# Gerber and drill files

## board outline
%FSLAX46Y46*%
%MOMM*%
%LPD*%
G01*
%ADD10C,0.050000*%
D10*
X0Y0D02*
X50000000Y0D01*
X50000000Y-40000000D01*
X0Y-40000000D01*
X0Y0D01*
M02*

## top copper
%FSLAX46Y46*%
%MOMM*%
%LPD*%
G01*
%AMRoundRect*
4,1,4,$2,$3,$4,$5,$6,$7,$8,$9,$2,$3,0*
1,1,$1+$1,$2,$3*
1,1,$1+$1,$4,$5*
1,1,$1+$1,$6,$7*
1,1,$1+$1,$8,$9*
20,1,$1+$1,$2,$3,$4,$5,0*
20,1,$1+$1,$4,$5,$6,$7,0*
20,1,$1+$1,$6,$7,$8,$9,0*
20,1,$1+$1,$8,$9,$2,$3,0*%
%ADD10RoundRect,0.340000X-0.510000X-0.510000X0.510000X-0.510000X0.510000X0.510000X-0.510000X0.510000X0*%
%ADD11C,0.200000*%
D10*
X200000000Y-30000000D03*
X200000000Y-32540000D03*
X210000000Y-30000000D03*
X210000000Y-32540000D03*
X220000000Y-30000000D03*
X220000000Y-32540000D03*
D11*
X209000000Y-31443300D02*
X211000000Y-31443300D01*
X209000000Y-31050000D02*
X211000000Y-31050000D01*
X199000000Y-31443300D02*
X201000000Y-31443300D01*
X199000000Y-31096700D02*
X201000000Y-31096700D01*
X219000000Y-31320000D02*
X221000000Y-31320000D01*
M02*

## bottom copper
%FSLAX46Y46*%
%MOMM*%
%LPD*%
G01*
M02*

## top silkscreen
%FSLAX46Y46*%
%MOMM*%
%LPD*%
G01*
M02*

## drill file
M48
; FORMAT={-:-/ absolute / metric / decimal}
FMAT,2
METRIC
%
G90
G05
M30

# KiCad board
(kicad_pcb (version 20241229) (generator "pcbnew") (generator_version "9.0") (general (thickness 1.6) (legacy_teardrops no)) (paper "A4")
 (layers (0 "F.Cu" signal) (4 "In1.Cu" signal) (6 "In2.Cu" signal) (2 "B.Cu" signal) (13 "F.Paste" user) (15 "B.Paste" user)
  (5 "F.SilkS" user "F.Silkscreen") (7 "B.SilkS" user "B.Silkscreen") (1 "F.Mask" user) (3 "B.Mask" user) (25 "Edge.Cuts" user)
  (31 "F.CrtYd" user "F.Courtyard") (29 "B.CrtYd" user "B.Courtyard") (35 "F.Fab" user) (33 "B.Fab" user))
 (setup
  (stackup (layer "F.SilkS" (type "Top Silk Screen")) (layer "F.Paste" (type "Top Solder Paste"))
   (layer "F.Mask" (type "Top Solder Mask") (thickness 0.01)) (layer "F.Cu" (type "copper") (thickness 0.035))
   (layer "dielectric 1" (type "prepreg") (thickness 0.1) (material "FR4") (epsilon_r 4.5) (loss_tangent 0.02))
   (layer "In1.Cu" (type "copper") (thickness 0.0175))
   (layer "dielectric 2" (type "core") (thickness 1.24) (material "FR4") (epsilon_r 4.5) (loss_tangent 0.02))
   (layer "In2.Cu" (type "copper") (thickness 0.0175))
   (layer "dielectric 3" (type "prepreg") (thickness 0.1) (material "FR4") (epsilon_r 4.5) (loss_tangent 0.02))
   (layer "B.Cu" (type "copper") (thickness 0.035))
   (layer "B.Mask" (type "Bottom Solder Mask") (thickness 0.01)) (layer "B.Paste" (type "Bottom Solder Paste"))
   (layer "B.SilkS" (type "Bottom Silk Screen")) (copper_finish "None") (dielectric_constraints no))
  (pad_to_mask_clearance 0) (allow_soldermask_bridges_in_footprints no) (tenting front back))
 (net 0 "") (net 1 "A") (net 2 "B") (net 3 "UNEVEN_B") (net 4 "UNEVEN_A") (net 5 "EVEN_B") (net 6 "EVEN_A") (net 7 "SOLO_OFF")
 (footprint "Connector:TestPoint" (layer "F.Cu") (at 200 30)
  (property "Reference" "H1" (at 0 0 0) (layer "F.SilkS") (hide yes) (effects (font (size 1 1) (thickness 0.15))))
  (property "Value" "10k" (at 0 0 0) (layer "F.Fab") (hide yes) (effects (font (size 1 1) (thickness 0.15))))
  (pad "1" smd roundrect (at 0 0) (size 1.7 1.7) (layers "F.Cu" "F.Paste" "F.Mask") (roundrect_rratio 0.2) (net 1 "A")))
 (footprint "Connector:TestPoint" (layer "F.Cu") (at 200 32.54)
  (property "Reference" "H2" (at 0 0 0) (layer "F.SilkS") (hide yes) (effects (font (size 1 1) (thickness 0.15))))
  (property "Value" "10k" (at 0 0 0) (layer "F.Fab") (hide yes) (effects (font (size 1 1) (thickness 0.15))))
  (pad "1" smd roundrect (at 0 0) (size 1.7 1.7) (layers "F.Cu" "F.Paste" "F.Mask") (roundrect_rratio 0.2) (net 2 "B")))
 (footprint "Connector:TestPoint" (layer "F.Cu") (at 210 30)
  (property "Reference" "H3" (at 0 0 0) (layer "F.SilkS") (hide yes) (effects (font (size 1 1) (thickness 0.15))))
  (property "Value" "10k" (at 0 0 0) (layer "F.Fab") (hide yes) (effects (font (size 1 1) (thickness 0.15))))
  (pad "1" smd roundrect (at 0 0) (size 1.7 1.7) (layers "F.Cu" "F.Paste" "F.Mask") (roundrect_rratio 0.2) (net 1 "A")))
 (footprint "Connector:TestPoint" (layer "F.Cu") (at 210 32.54)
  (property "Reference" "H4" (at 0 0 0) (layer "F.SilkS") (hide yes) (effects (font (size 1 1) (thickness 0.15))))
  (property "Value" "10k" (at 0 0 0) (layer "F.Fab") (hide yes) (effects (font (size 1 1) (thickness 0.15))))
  (pad "1" smd roundrect (at 0 0) (size 1.7 1.7) (layers "F.Cu" "F.Paste" "F.Mask") (roundrect_rratio 0.2) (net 2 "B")))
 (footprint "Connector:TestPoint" (layer "F.Cu") (at 220 30)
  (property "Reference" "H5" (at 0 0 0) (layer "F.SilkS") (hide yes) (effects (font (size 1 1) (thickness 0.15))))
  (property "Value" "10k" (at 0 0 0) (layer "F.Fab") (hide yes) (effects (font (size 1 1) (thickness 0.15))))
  (pad "1" smd roundrect (at 0 0) (size 1.7 1.7) (layers "F.Cu" "F.Paste" "F.Mask") (roundrect_rratio 0.2) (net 1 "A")))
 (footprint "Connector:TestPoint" (layer "F.Cu") (at 220 32.54)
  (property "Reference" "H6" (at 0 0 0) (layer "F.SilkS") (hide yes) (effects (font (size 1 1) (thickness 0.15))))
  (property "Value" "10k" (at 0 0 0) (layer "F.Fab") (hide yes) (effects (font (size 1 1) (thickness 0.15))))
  (pad "1" smd roundrect (at 0 0) (size 1.7 1.7) (layers "F.Cu" "F.Paste" "F.Mask") (roundrect_rratio 0.2) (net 2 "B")))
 (segment (start 209 31.4433) (end 211 31.4433) (width 0.2) (layer "F.Cu") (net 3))
 (segment (start 209 31.05) (end 211 31.05) (width 0.2) (layer "F.Cu") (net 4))
 (segment (start 199 31.4433) (end 201 31.4433) (width 0.2) (layer "F.Cu") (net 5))
 (segment (start 199 31.0967) (end 201 31.0967) (width 0.2) (layer "F.Cu") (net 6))
 (segment (start 219 31.32) (end 221 31.32) (width 0.2) (layer "F.Cu") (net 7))
 (gr_rect (start 0 0) (end 50 40) (stroke (width 0.05) (type default)) (fill no) (layer "Edge.Cuts")))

